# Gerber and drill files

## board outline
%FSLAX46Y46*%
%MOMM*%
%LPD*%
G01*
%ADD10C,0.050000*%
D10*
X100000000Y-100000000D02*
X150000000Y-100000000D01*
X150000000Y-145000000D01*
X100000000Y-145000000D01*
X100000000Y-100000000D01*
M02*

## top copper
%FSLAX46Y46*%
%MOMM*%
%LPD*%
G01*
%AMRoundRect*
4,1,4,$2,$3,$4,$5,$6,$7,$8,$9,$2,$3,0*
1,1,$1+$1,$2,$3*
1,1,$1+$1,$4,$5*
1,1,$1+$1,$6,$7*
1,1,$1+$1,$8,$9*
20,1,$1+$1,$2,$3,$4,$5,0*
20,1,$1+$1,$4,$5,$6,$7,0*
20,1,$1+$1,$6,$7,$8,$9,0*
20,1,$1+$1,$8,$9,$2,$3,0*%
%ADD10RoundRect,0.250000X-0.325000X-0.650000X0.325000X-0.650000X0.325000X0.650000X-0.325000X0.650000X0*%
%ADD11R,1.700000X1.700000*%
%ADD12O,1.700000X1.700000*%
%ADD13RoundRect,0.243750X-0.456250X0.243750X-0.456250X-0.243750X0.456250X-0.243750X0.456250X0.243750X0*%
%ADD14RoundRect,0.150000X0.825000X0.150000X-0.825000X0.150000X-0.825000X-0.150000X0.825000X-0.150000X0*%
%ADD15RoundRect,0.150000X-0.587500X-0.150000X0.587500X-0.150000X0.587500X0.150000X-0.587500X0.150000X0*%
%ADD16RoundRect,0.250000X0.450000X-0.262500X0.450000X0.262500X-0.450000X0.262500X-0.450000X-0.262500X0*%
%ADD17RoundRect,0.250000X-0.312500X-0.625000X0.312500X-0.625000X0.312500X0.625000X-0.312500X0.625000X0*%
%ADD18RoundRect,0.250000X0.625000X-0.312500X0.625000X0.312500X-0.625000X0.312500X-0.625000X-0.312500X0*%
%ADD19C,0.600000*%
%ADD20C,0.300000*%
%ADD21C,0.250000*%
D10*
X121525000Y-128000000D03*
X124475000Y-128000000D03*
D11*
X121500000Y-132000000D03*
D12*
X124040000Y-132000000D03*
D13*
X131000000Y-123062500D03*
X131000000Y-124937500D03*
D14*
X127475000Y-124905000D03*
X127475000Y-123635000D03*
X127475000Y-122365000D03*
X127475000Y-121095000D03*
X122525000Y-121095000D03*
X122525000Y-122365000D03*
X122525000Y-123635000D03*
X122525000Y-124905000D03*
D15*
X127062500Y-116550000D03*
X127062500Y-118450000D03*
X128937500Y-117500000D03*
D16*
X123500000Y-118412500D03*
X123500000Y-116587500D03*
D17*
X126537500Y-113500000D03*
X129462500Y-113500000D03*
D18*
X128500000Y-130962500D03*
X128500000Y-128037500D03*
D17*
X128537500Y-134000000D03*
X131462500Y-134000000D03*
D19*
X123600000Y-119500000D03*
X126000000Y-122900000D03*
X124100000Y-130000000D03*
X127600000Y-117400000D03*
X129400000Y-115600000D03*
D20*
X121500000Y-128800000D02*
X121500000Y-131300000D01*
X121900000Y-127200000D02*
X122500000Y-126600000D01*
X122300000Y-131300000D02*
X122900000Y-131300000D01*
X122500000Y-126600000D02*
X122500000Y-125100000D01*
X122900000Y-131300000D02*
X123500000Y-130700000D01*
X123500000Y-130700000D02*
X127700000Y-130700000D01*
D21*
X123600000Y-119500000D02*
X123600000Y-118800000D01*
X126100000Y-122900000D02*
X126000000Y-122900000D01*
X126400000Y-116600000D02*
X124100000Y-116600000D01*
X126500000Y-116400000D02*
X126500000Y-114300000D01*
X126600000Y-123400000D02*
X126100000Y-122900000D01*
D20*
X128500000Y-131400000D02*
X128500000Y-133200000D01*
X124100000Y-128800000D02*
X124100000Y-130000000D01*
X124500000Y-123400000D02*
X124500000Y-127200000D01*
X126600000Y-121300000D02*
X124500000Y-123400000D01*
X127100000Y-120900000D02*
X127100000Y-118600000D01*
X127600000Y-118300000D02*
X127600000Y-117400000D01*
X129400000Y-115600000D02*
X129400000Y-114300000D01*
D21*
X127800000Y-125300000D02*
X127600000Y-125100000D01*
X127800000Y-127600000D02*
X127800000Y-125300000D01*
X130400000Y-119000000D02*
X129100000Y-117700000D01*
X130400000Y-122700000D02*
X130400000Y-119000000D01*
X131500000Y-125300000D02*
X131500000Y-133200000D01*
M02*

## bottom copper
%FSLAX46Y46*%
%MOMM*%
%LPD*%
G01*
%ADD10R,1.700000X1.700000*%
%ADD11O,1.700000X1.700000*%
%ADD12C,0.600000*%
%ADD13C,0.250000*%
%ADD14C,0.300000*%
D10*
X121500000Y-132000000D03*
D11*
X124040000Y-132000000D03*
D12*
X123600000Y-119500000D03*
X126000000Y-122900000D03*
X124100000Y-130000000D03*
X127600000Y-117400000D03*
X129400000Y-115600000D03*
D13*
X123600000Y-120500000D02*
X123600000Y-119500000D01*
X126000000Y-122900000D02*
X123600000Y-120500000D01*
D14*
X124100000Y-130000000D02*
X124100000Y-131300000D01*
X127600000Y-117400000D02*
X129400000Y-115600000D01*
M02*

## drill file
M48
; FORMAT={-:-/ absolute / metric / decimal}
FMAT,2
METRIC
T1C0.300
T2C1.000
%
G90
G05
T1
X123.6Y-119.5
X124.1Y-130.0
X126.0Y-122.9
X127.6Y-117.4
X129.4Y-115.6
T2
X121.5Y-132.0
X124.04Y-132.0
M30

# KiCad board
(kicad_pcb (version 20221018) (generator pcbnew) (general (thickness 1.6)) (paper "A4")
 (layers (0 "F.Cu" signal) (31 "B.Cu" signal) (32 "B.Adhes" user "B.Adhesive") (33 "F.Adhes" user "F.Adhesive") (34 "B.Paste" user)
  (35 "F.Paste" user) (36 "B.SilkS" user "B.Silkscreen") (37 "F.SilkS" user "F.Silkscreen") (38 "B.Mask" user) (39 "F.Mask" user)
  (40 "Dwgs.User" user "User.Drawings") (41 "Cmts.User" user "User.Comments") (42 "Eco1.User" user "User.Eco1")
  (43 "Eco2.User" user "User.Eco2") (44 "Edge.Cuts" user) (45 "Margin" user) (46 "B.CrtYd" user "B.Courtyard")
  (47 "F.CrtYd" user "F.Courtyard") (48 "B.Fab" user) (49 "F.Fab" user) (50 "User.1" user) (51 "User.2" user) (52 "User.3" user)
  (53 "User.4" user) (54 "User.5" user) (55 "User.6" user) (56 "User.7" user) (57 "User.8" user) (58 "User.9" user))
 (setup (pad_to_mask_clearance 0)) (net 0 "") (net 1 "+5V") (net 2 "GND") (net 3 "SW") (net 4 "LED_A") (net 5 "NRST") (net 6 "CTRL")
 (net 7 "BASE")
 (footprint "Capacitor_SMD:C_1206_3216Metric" (layer "F.Cu") (at 123 128)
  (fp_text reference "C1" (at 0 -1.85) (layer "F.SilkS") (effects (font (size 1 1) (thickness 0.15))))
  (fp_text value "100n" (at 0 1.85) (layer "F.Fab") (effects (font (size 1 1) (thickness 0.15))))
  (pad "1" smd roundrect (at -1.475 0) (size 1.15 1.8) (layers "F.Cu" "F.Paste" "F.Mask") (roundrect_rratio 0.217391) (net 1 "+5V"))
  (pad "2" smd roundrect (at 1.475 0) (size 1.15 1.8) (layers "F.Cu" "F.Paste" "F.Mask") (roundrect_rratio 0.217391) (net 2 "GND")))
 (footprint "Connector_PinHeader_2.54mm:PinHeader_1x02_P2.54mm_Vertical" (layer "F.Cu") (at 121.5 132 90)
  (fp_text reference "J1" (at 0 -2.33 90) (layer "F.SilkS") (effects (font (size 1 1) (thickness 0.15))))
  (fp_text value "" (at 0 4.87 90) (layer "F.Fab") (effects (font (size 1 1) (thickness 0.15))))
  (pad "1" thru_hole rect (at 0 0 90) (size 1.7 1.7) (drill 1) (layers "*.Cu" "*.Mask") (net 1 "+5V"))
  (pad "2" thru_hole oval (at 0 2.54 90) (size 1.7 1.7) (drill 1) (layers "*.Cu" "*.Mask") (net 2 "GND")))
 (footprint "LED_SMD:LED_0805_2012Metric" (layer "F.Cu") (at 131 124 -90)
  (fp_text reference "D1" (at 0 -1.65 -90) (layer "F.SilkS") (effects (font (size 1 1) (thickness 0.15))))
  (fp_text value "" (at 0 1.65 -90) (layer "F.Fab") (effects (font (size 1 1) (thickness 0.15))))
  (pad "1" smd roundrect (at -0.9375 0 270) (size 0.975 1.4) (layers "F.Cu" "F.Paste" "F.Mask") (roundrect_rratio 0.25) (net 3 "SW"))
  (pad "2" smd roundrect (at 0.9375 0 270) (size 0.975 1.4) (layers "F.Cu" "F.Paste" "F.Mask") (roundrect_rratio 0.25) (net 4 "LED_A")))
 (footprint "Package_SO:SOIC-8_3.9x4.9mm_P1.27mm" (layer "F.Cu") (at 125 123 180)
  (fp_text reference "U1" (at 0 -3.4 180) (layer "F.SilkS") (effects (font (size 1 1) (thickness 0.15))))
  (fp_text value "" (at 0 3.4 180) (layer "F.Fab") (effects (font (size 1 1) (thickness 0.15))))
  (pad "1" smd roundrect (at -2.475 -1.905 180) (size 1.95 0.6) (layers "F.Cu" "F.Paste" "F.Mask") (roundrect_rratio 0.25) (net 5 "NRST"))
  (pad "2" smd roundrect (at -2.475 -0.635 180) (size 1.95 0.6) (layers "F.Cu" "F.Paste" "F.Mask") (roundrect_rratio 0.25) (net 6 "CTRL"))
  (pad "3" smd roundrect (at -2.475 0.635 180) (size 1.95 0.6) (layers "F.Cu" "F.Paste" "F.Mask") (roundrect_rratio 0.25))
  (pad "4" smd roundrect (at -2.475 1.905 180) (size 1.95 0.6) (layers "F.Cu" "F.Paste" "F.Mask") (roundrect_rratio 0.25) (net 2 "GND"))
  (pad "5" smd roundrect (at 2.475 1.905 180) (size 1.95 0.6) (layers "F.Cu" "F.Paste" "F.Mask") (roundrect_rratio 0.25))
  (pad "6" smd roundrect (at 2.475 0.635 180) (size 1.95 0.6) (layers "F.Cu" "F.Paste" "F.Mask") (roundrect_rratio 0.25))
  (pad "7" smd roundrect (at 2.475 -0.635 180) (size 1.95 0.6) (layers "F.Cu" "F.Paste" "F.Mask") (roundrect_rratio 0.25))
  (pad "8" smd roundrect (at 2.475 -1.905 180) (size 1.95 0.6) (layers "F.Cu" "F.Paste" "F.Mask") (roundrect_rratio 0.25) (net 1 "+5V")))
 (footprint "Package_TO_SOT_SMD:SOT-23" (layer "F.Cu") (at 128 117.5)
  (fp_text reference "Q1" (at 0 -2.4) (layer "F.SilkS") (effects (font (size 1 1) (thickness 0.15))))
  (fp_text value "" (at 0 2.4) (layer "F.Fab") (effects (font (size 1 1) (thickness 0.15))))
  (pad "1" smd roundrect (at -0.9375 -0.95) (size 1.475 0.6) (layers "F.Cu" "F.Paste" "F.Mask") (roundrect_rratio 0.25) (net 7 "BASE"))
  (pad "2" smd roundrect (at -0.9375 0.95) (size 1.475 0.6) (layers "F.Cu" "F.Paste" "F.Mask") (roundrect_rratio 0.25) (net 2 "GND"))
  (pad "3" smd roundrect (at 0.9375 0) (size 1.475 0.6) (layers "F.Cu" "F.Paste" "F.Mask") (roundrect_rratio 0.25) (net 3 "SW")))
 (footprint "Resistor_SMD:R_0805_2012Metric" (layer "F.Cu") (at 123.5 117.5 90)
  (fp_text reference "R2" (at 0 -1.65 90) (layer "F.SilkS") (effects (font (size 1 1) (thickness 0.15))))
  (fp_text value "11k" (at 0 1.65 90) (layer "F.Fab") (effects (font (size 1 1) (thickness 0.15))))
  (pad "1" smd roundrect (at -0.9125 0 90) (size 1.025 1.4) (layers "F.Cu" "F.Paste" "F.Mask") (roundrect_rratio 0.243902) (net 6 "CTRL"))
  (pad "2" smd roundrect (at 0.9125 0 90) (size 1.025 1.4) (layers "F.Cu" "F.Paste" "F.Mask") (roundrect_rratio 0.243902) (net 7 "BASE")))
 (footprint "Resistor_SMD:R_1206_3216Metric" (layer "F.Cu") (at 128 113.5)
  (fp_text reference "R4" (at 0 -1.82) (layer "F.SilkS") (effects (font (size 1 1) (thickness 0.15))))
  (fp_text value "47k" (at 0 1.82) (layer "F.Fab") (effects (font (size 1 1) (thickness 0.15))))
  (pad "1" smd roundrect (at -1.4625 0) (size 1.125 1.75) (layers "F.Cu" "F.Paste" "F.Mask") (roundrect_rratio 0.222222) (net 7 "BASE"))
  (pad "2" smd roundrect (at 1.4625 0) (size 1.125 1.75) (layers "F.Cu" "F.Paste" "F.Mask") (roundrect_rratio 0.222222) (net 2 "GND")))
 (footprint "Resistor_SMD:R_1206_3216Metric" (layer "F.Cu") (at 128.5 129.5 90)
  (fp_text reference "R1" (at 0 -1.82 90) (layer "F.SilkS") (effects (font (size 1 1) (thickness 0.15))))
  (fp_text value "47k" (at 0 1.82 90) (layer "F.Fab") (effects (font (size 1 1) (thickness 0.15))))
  (pad "1" smd roundrect (at -1.4625 0 90) (size 1.125 1.75) (layers "F.Cu" "F.Paste" "F.Mask") (roundrect_rratio 0.222222) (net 1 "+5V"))
  (pad "2" smd roundrect (at 1.4625 0 90) (size 1.125 1.75) (layers "F.Cu" "F.Paste" "F.Mask") (roundrect_rratio 0.222222) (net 5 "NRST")))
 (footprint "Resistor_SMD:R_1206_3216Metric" (layer "F.Cu") (at 130 134)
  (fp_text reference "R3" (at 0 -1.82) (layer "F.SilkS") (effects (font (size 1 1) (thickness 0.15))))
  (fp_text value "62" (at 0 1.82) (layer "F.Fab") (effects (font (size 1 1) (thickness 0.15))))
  (pad "1" smd roundrect (at -1.4625 0) (size 1.125 1.75) (layers "F.Cu" "F.Paste" "F.Mask") (roundrect_rratio 0.222222) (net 1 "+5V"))
  (pad "2" smd roundrect (at 1.4625 0) (size 1.125 1.75) (layers "F.Cu" "F.Paste" "F.Mask") (roundrect_rratio 0.222222) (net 4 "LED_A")))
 (gr_rect (start 100 100) (end 150 145) (stroke (width 0.05) (type default)) (fill none) (layer "Edge.Cuts"))
 (segment (start 121.5 128.8) (end 121.5 131.3) (width 0.3) (layer "F.Cu") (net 1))
 (segment (start 121.9 127.2) (end 122.5 126.6) (width 0.3) (layer "F.Cu") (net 1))
 (segment (start 122.3 131.3) (end 122.9 131.3) (width 0.3) (layer "F.Cu") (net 1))
 (segment (start 122.5 126.6) (end 122.5 125.1) (width 0.3) (layer "F.Cu") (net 1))
 (segment (start 122.9 131.3) (end 123.5 130.7) (width 0.3) (layer "F.Cu") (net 1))
 (segment (start 123.5 130.7) (end 127.7 130.7) (width 0.3) (layer "F.Cu") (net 1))
 (segment (start 123.6 119.5) (end 123.6 118.8) (width 0.25) (layer "F.Cu") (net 6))
 (segment (start 126.1 122.9) (end 126 122.9) (width 0.25) (layer "F.Cu") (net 6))
 (segment (start 126.4 116.6) (end 124.1 116.6) (width 0.25) (layer "F.Cu") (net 7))
 (segment (start 126.5 116.4) (end 126.5 114.3) (width 0.25) (layer "F.Cu") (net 7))
 (segment (start 126.6 123.4) (end 126.1 122.9) (width 0.25) (layer "F.Cu") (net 6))
 (segment (start 128.5 131.4) (end 128.5 133.2) (width 0.3) (layer "F.Cu") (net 1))
 (via (at 123.6 119.5) (size 0.6) (drill 0.3) (layers "F.Cu" "B.Cu") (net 6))
 (via (at 126 122.9) (size 0.6) (drill 0.3) (layers "F.Cu" "B.Cu") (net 6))
 (segment (start 123.6 120.5) (end 123.6 119.5) (width 0.25) (layer "B.Cu") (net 6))
 (segment (start 124.1 128.8) (end 124.1 130) (width 0.3) (layer "F.Cu") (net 2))
 (segment (start 124.5 123.4) (end 124.5 127.2) (width 0.3) (layer "F.Cu") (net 2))
 (segment (start 126 122.9) (end 123.6 120.5) (width 0.25) (layer "B.Cu") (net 6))
 (segment (start 126.6 121.3) (end 124.5 123.4) (width 0.3) (layer "F.Cu") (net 2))
 (segment (start 127.1 120.9) (end 127.1 118.6) (width 0.3) (layer "F.Cu") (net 2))
 (segment (start 127.6 118.3) (end 127.6 117.4) (width 0.3) (layer "F.Cu") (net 2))
 (segment (start 129.4 115.6) (end 129.4 114.3) (width 0.3) (layer "F.Cu") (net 2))
 (via (at 124.1 130) (size 0.6) (drill 0.3) (layers "F.Cu" "B.Cu") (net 2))
 (via (at 127.6 117.4) (size 0.6) (drill 0.3) (layers "F.Cu" "B.Cu") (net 2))
 (via (at 129.4 115.6) (size 0.6) (drill 0.3) (layers "F.Cu" "B.Cu") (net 2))
 (segment (start 124.1 130) (end 124.1 131.3) (width 0.3) (layer "B.Cu") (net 2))
 (segment (start 127.6 117.4) (end 129.4 115.6) (width 0.3) (layer "B.Cu") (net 2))
 (segment (start 127.8 125.3) (end 127.6 125.1) (width 0.25) (layer "F.Cu") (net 5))
 (segment (start 127.8 127.6) (end 127.8 125.3) (width 0.25) (layer "F.Cu") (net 5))
 (segment (start 130.4 119) (end 129.1 117.7) (width 0.25) (layer "F.Cu") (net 3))
 (segment (start 130.4 122.7) (end 130.4 119) (width 0.25) (layer "F.Cu") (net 3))
 (segment (start 131.5 125.3) (end 131.5 133.2) (width 0.25) (layer "F.Cu") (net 4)))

